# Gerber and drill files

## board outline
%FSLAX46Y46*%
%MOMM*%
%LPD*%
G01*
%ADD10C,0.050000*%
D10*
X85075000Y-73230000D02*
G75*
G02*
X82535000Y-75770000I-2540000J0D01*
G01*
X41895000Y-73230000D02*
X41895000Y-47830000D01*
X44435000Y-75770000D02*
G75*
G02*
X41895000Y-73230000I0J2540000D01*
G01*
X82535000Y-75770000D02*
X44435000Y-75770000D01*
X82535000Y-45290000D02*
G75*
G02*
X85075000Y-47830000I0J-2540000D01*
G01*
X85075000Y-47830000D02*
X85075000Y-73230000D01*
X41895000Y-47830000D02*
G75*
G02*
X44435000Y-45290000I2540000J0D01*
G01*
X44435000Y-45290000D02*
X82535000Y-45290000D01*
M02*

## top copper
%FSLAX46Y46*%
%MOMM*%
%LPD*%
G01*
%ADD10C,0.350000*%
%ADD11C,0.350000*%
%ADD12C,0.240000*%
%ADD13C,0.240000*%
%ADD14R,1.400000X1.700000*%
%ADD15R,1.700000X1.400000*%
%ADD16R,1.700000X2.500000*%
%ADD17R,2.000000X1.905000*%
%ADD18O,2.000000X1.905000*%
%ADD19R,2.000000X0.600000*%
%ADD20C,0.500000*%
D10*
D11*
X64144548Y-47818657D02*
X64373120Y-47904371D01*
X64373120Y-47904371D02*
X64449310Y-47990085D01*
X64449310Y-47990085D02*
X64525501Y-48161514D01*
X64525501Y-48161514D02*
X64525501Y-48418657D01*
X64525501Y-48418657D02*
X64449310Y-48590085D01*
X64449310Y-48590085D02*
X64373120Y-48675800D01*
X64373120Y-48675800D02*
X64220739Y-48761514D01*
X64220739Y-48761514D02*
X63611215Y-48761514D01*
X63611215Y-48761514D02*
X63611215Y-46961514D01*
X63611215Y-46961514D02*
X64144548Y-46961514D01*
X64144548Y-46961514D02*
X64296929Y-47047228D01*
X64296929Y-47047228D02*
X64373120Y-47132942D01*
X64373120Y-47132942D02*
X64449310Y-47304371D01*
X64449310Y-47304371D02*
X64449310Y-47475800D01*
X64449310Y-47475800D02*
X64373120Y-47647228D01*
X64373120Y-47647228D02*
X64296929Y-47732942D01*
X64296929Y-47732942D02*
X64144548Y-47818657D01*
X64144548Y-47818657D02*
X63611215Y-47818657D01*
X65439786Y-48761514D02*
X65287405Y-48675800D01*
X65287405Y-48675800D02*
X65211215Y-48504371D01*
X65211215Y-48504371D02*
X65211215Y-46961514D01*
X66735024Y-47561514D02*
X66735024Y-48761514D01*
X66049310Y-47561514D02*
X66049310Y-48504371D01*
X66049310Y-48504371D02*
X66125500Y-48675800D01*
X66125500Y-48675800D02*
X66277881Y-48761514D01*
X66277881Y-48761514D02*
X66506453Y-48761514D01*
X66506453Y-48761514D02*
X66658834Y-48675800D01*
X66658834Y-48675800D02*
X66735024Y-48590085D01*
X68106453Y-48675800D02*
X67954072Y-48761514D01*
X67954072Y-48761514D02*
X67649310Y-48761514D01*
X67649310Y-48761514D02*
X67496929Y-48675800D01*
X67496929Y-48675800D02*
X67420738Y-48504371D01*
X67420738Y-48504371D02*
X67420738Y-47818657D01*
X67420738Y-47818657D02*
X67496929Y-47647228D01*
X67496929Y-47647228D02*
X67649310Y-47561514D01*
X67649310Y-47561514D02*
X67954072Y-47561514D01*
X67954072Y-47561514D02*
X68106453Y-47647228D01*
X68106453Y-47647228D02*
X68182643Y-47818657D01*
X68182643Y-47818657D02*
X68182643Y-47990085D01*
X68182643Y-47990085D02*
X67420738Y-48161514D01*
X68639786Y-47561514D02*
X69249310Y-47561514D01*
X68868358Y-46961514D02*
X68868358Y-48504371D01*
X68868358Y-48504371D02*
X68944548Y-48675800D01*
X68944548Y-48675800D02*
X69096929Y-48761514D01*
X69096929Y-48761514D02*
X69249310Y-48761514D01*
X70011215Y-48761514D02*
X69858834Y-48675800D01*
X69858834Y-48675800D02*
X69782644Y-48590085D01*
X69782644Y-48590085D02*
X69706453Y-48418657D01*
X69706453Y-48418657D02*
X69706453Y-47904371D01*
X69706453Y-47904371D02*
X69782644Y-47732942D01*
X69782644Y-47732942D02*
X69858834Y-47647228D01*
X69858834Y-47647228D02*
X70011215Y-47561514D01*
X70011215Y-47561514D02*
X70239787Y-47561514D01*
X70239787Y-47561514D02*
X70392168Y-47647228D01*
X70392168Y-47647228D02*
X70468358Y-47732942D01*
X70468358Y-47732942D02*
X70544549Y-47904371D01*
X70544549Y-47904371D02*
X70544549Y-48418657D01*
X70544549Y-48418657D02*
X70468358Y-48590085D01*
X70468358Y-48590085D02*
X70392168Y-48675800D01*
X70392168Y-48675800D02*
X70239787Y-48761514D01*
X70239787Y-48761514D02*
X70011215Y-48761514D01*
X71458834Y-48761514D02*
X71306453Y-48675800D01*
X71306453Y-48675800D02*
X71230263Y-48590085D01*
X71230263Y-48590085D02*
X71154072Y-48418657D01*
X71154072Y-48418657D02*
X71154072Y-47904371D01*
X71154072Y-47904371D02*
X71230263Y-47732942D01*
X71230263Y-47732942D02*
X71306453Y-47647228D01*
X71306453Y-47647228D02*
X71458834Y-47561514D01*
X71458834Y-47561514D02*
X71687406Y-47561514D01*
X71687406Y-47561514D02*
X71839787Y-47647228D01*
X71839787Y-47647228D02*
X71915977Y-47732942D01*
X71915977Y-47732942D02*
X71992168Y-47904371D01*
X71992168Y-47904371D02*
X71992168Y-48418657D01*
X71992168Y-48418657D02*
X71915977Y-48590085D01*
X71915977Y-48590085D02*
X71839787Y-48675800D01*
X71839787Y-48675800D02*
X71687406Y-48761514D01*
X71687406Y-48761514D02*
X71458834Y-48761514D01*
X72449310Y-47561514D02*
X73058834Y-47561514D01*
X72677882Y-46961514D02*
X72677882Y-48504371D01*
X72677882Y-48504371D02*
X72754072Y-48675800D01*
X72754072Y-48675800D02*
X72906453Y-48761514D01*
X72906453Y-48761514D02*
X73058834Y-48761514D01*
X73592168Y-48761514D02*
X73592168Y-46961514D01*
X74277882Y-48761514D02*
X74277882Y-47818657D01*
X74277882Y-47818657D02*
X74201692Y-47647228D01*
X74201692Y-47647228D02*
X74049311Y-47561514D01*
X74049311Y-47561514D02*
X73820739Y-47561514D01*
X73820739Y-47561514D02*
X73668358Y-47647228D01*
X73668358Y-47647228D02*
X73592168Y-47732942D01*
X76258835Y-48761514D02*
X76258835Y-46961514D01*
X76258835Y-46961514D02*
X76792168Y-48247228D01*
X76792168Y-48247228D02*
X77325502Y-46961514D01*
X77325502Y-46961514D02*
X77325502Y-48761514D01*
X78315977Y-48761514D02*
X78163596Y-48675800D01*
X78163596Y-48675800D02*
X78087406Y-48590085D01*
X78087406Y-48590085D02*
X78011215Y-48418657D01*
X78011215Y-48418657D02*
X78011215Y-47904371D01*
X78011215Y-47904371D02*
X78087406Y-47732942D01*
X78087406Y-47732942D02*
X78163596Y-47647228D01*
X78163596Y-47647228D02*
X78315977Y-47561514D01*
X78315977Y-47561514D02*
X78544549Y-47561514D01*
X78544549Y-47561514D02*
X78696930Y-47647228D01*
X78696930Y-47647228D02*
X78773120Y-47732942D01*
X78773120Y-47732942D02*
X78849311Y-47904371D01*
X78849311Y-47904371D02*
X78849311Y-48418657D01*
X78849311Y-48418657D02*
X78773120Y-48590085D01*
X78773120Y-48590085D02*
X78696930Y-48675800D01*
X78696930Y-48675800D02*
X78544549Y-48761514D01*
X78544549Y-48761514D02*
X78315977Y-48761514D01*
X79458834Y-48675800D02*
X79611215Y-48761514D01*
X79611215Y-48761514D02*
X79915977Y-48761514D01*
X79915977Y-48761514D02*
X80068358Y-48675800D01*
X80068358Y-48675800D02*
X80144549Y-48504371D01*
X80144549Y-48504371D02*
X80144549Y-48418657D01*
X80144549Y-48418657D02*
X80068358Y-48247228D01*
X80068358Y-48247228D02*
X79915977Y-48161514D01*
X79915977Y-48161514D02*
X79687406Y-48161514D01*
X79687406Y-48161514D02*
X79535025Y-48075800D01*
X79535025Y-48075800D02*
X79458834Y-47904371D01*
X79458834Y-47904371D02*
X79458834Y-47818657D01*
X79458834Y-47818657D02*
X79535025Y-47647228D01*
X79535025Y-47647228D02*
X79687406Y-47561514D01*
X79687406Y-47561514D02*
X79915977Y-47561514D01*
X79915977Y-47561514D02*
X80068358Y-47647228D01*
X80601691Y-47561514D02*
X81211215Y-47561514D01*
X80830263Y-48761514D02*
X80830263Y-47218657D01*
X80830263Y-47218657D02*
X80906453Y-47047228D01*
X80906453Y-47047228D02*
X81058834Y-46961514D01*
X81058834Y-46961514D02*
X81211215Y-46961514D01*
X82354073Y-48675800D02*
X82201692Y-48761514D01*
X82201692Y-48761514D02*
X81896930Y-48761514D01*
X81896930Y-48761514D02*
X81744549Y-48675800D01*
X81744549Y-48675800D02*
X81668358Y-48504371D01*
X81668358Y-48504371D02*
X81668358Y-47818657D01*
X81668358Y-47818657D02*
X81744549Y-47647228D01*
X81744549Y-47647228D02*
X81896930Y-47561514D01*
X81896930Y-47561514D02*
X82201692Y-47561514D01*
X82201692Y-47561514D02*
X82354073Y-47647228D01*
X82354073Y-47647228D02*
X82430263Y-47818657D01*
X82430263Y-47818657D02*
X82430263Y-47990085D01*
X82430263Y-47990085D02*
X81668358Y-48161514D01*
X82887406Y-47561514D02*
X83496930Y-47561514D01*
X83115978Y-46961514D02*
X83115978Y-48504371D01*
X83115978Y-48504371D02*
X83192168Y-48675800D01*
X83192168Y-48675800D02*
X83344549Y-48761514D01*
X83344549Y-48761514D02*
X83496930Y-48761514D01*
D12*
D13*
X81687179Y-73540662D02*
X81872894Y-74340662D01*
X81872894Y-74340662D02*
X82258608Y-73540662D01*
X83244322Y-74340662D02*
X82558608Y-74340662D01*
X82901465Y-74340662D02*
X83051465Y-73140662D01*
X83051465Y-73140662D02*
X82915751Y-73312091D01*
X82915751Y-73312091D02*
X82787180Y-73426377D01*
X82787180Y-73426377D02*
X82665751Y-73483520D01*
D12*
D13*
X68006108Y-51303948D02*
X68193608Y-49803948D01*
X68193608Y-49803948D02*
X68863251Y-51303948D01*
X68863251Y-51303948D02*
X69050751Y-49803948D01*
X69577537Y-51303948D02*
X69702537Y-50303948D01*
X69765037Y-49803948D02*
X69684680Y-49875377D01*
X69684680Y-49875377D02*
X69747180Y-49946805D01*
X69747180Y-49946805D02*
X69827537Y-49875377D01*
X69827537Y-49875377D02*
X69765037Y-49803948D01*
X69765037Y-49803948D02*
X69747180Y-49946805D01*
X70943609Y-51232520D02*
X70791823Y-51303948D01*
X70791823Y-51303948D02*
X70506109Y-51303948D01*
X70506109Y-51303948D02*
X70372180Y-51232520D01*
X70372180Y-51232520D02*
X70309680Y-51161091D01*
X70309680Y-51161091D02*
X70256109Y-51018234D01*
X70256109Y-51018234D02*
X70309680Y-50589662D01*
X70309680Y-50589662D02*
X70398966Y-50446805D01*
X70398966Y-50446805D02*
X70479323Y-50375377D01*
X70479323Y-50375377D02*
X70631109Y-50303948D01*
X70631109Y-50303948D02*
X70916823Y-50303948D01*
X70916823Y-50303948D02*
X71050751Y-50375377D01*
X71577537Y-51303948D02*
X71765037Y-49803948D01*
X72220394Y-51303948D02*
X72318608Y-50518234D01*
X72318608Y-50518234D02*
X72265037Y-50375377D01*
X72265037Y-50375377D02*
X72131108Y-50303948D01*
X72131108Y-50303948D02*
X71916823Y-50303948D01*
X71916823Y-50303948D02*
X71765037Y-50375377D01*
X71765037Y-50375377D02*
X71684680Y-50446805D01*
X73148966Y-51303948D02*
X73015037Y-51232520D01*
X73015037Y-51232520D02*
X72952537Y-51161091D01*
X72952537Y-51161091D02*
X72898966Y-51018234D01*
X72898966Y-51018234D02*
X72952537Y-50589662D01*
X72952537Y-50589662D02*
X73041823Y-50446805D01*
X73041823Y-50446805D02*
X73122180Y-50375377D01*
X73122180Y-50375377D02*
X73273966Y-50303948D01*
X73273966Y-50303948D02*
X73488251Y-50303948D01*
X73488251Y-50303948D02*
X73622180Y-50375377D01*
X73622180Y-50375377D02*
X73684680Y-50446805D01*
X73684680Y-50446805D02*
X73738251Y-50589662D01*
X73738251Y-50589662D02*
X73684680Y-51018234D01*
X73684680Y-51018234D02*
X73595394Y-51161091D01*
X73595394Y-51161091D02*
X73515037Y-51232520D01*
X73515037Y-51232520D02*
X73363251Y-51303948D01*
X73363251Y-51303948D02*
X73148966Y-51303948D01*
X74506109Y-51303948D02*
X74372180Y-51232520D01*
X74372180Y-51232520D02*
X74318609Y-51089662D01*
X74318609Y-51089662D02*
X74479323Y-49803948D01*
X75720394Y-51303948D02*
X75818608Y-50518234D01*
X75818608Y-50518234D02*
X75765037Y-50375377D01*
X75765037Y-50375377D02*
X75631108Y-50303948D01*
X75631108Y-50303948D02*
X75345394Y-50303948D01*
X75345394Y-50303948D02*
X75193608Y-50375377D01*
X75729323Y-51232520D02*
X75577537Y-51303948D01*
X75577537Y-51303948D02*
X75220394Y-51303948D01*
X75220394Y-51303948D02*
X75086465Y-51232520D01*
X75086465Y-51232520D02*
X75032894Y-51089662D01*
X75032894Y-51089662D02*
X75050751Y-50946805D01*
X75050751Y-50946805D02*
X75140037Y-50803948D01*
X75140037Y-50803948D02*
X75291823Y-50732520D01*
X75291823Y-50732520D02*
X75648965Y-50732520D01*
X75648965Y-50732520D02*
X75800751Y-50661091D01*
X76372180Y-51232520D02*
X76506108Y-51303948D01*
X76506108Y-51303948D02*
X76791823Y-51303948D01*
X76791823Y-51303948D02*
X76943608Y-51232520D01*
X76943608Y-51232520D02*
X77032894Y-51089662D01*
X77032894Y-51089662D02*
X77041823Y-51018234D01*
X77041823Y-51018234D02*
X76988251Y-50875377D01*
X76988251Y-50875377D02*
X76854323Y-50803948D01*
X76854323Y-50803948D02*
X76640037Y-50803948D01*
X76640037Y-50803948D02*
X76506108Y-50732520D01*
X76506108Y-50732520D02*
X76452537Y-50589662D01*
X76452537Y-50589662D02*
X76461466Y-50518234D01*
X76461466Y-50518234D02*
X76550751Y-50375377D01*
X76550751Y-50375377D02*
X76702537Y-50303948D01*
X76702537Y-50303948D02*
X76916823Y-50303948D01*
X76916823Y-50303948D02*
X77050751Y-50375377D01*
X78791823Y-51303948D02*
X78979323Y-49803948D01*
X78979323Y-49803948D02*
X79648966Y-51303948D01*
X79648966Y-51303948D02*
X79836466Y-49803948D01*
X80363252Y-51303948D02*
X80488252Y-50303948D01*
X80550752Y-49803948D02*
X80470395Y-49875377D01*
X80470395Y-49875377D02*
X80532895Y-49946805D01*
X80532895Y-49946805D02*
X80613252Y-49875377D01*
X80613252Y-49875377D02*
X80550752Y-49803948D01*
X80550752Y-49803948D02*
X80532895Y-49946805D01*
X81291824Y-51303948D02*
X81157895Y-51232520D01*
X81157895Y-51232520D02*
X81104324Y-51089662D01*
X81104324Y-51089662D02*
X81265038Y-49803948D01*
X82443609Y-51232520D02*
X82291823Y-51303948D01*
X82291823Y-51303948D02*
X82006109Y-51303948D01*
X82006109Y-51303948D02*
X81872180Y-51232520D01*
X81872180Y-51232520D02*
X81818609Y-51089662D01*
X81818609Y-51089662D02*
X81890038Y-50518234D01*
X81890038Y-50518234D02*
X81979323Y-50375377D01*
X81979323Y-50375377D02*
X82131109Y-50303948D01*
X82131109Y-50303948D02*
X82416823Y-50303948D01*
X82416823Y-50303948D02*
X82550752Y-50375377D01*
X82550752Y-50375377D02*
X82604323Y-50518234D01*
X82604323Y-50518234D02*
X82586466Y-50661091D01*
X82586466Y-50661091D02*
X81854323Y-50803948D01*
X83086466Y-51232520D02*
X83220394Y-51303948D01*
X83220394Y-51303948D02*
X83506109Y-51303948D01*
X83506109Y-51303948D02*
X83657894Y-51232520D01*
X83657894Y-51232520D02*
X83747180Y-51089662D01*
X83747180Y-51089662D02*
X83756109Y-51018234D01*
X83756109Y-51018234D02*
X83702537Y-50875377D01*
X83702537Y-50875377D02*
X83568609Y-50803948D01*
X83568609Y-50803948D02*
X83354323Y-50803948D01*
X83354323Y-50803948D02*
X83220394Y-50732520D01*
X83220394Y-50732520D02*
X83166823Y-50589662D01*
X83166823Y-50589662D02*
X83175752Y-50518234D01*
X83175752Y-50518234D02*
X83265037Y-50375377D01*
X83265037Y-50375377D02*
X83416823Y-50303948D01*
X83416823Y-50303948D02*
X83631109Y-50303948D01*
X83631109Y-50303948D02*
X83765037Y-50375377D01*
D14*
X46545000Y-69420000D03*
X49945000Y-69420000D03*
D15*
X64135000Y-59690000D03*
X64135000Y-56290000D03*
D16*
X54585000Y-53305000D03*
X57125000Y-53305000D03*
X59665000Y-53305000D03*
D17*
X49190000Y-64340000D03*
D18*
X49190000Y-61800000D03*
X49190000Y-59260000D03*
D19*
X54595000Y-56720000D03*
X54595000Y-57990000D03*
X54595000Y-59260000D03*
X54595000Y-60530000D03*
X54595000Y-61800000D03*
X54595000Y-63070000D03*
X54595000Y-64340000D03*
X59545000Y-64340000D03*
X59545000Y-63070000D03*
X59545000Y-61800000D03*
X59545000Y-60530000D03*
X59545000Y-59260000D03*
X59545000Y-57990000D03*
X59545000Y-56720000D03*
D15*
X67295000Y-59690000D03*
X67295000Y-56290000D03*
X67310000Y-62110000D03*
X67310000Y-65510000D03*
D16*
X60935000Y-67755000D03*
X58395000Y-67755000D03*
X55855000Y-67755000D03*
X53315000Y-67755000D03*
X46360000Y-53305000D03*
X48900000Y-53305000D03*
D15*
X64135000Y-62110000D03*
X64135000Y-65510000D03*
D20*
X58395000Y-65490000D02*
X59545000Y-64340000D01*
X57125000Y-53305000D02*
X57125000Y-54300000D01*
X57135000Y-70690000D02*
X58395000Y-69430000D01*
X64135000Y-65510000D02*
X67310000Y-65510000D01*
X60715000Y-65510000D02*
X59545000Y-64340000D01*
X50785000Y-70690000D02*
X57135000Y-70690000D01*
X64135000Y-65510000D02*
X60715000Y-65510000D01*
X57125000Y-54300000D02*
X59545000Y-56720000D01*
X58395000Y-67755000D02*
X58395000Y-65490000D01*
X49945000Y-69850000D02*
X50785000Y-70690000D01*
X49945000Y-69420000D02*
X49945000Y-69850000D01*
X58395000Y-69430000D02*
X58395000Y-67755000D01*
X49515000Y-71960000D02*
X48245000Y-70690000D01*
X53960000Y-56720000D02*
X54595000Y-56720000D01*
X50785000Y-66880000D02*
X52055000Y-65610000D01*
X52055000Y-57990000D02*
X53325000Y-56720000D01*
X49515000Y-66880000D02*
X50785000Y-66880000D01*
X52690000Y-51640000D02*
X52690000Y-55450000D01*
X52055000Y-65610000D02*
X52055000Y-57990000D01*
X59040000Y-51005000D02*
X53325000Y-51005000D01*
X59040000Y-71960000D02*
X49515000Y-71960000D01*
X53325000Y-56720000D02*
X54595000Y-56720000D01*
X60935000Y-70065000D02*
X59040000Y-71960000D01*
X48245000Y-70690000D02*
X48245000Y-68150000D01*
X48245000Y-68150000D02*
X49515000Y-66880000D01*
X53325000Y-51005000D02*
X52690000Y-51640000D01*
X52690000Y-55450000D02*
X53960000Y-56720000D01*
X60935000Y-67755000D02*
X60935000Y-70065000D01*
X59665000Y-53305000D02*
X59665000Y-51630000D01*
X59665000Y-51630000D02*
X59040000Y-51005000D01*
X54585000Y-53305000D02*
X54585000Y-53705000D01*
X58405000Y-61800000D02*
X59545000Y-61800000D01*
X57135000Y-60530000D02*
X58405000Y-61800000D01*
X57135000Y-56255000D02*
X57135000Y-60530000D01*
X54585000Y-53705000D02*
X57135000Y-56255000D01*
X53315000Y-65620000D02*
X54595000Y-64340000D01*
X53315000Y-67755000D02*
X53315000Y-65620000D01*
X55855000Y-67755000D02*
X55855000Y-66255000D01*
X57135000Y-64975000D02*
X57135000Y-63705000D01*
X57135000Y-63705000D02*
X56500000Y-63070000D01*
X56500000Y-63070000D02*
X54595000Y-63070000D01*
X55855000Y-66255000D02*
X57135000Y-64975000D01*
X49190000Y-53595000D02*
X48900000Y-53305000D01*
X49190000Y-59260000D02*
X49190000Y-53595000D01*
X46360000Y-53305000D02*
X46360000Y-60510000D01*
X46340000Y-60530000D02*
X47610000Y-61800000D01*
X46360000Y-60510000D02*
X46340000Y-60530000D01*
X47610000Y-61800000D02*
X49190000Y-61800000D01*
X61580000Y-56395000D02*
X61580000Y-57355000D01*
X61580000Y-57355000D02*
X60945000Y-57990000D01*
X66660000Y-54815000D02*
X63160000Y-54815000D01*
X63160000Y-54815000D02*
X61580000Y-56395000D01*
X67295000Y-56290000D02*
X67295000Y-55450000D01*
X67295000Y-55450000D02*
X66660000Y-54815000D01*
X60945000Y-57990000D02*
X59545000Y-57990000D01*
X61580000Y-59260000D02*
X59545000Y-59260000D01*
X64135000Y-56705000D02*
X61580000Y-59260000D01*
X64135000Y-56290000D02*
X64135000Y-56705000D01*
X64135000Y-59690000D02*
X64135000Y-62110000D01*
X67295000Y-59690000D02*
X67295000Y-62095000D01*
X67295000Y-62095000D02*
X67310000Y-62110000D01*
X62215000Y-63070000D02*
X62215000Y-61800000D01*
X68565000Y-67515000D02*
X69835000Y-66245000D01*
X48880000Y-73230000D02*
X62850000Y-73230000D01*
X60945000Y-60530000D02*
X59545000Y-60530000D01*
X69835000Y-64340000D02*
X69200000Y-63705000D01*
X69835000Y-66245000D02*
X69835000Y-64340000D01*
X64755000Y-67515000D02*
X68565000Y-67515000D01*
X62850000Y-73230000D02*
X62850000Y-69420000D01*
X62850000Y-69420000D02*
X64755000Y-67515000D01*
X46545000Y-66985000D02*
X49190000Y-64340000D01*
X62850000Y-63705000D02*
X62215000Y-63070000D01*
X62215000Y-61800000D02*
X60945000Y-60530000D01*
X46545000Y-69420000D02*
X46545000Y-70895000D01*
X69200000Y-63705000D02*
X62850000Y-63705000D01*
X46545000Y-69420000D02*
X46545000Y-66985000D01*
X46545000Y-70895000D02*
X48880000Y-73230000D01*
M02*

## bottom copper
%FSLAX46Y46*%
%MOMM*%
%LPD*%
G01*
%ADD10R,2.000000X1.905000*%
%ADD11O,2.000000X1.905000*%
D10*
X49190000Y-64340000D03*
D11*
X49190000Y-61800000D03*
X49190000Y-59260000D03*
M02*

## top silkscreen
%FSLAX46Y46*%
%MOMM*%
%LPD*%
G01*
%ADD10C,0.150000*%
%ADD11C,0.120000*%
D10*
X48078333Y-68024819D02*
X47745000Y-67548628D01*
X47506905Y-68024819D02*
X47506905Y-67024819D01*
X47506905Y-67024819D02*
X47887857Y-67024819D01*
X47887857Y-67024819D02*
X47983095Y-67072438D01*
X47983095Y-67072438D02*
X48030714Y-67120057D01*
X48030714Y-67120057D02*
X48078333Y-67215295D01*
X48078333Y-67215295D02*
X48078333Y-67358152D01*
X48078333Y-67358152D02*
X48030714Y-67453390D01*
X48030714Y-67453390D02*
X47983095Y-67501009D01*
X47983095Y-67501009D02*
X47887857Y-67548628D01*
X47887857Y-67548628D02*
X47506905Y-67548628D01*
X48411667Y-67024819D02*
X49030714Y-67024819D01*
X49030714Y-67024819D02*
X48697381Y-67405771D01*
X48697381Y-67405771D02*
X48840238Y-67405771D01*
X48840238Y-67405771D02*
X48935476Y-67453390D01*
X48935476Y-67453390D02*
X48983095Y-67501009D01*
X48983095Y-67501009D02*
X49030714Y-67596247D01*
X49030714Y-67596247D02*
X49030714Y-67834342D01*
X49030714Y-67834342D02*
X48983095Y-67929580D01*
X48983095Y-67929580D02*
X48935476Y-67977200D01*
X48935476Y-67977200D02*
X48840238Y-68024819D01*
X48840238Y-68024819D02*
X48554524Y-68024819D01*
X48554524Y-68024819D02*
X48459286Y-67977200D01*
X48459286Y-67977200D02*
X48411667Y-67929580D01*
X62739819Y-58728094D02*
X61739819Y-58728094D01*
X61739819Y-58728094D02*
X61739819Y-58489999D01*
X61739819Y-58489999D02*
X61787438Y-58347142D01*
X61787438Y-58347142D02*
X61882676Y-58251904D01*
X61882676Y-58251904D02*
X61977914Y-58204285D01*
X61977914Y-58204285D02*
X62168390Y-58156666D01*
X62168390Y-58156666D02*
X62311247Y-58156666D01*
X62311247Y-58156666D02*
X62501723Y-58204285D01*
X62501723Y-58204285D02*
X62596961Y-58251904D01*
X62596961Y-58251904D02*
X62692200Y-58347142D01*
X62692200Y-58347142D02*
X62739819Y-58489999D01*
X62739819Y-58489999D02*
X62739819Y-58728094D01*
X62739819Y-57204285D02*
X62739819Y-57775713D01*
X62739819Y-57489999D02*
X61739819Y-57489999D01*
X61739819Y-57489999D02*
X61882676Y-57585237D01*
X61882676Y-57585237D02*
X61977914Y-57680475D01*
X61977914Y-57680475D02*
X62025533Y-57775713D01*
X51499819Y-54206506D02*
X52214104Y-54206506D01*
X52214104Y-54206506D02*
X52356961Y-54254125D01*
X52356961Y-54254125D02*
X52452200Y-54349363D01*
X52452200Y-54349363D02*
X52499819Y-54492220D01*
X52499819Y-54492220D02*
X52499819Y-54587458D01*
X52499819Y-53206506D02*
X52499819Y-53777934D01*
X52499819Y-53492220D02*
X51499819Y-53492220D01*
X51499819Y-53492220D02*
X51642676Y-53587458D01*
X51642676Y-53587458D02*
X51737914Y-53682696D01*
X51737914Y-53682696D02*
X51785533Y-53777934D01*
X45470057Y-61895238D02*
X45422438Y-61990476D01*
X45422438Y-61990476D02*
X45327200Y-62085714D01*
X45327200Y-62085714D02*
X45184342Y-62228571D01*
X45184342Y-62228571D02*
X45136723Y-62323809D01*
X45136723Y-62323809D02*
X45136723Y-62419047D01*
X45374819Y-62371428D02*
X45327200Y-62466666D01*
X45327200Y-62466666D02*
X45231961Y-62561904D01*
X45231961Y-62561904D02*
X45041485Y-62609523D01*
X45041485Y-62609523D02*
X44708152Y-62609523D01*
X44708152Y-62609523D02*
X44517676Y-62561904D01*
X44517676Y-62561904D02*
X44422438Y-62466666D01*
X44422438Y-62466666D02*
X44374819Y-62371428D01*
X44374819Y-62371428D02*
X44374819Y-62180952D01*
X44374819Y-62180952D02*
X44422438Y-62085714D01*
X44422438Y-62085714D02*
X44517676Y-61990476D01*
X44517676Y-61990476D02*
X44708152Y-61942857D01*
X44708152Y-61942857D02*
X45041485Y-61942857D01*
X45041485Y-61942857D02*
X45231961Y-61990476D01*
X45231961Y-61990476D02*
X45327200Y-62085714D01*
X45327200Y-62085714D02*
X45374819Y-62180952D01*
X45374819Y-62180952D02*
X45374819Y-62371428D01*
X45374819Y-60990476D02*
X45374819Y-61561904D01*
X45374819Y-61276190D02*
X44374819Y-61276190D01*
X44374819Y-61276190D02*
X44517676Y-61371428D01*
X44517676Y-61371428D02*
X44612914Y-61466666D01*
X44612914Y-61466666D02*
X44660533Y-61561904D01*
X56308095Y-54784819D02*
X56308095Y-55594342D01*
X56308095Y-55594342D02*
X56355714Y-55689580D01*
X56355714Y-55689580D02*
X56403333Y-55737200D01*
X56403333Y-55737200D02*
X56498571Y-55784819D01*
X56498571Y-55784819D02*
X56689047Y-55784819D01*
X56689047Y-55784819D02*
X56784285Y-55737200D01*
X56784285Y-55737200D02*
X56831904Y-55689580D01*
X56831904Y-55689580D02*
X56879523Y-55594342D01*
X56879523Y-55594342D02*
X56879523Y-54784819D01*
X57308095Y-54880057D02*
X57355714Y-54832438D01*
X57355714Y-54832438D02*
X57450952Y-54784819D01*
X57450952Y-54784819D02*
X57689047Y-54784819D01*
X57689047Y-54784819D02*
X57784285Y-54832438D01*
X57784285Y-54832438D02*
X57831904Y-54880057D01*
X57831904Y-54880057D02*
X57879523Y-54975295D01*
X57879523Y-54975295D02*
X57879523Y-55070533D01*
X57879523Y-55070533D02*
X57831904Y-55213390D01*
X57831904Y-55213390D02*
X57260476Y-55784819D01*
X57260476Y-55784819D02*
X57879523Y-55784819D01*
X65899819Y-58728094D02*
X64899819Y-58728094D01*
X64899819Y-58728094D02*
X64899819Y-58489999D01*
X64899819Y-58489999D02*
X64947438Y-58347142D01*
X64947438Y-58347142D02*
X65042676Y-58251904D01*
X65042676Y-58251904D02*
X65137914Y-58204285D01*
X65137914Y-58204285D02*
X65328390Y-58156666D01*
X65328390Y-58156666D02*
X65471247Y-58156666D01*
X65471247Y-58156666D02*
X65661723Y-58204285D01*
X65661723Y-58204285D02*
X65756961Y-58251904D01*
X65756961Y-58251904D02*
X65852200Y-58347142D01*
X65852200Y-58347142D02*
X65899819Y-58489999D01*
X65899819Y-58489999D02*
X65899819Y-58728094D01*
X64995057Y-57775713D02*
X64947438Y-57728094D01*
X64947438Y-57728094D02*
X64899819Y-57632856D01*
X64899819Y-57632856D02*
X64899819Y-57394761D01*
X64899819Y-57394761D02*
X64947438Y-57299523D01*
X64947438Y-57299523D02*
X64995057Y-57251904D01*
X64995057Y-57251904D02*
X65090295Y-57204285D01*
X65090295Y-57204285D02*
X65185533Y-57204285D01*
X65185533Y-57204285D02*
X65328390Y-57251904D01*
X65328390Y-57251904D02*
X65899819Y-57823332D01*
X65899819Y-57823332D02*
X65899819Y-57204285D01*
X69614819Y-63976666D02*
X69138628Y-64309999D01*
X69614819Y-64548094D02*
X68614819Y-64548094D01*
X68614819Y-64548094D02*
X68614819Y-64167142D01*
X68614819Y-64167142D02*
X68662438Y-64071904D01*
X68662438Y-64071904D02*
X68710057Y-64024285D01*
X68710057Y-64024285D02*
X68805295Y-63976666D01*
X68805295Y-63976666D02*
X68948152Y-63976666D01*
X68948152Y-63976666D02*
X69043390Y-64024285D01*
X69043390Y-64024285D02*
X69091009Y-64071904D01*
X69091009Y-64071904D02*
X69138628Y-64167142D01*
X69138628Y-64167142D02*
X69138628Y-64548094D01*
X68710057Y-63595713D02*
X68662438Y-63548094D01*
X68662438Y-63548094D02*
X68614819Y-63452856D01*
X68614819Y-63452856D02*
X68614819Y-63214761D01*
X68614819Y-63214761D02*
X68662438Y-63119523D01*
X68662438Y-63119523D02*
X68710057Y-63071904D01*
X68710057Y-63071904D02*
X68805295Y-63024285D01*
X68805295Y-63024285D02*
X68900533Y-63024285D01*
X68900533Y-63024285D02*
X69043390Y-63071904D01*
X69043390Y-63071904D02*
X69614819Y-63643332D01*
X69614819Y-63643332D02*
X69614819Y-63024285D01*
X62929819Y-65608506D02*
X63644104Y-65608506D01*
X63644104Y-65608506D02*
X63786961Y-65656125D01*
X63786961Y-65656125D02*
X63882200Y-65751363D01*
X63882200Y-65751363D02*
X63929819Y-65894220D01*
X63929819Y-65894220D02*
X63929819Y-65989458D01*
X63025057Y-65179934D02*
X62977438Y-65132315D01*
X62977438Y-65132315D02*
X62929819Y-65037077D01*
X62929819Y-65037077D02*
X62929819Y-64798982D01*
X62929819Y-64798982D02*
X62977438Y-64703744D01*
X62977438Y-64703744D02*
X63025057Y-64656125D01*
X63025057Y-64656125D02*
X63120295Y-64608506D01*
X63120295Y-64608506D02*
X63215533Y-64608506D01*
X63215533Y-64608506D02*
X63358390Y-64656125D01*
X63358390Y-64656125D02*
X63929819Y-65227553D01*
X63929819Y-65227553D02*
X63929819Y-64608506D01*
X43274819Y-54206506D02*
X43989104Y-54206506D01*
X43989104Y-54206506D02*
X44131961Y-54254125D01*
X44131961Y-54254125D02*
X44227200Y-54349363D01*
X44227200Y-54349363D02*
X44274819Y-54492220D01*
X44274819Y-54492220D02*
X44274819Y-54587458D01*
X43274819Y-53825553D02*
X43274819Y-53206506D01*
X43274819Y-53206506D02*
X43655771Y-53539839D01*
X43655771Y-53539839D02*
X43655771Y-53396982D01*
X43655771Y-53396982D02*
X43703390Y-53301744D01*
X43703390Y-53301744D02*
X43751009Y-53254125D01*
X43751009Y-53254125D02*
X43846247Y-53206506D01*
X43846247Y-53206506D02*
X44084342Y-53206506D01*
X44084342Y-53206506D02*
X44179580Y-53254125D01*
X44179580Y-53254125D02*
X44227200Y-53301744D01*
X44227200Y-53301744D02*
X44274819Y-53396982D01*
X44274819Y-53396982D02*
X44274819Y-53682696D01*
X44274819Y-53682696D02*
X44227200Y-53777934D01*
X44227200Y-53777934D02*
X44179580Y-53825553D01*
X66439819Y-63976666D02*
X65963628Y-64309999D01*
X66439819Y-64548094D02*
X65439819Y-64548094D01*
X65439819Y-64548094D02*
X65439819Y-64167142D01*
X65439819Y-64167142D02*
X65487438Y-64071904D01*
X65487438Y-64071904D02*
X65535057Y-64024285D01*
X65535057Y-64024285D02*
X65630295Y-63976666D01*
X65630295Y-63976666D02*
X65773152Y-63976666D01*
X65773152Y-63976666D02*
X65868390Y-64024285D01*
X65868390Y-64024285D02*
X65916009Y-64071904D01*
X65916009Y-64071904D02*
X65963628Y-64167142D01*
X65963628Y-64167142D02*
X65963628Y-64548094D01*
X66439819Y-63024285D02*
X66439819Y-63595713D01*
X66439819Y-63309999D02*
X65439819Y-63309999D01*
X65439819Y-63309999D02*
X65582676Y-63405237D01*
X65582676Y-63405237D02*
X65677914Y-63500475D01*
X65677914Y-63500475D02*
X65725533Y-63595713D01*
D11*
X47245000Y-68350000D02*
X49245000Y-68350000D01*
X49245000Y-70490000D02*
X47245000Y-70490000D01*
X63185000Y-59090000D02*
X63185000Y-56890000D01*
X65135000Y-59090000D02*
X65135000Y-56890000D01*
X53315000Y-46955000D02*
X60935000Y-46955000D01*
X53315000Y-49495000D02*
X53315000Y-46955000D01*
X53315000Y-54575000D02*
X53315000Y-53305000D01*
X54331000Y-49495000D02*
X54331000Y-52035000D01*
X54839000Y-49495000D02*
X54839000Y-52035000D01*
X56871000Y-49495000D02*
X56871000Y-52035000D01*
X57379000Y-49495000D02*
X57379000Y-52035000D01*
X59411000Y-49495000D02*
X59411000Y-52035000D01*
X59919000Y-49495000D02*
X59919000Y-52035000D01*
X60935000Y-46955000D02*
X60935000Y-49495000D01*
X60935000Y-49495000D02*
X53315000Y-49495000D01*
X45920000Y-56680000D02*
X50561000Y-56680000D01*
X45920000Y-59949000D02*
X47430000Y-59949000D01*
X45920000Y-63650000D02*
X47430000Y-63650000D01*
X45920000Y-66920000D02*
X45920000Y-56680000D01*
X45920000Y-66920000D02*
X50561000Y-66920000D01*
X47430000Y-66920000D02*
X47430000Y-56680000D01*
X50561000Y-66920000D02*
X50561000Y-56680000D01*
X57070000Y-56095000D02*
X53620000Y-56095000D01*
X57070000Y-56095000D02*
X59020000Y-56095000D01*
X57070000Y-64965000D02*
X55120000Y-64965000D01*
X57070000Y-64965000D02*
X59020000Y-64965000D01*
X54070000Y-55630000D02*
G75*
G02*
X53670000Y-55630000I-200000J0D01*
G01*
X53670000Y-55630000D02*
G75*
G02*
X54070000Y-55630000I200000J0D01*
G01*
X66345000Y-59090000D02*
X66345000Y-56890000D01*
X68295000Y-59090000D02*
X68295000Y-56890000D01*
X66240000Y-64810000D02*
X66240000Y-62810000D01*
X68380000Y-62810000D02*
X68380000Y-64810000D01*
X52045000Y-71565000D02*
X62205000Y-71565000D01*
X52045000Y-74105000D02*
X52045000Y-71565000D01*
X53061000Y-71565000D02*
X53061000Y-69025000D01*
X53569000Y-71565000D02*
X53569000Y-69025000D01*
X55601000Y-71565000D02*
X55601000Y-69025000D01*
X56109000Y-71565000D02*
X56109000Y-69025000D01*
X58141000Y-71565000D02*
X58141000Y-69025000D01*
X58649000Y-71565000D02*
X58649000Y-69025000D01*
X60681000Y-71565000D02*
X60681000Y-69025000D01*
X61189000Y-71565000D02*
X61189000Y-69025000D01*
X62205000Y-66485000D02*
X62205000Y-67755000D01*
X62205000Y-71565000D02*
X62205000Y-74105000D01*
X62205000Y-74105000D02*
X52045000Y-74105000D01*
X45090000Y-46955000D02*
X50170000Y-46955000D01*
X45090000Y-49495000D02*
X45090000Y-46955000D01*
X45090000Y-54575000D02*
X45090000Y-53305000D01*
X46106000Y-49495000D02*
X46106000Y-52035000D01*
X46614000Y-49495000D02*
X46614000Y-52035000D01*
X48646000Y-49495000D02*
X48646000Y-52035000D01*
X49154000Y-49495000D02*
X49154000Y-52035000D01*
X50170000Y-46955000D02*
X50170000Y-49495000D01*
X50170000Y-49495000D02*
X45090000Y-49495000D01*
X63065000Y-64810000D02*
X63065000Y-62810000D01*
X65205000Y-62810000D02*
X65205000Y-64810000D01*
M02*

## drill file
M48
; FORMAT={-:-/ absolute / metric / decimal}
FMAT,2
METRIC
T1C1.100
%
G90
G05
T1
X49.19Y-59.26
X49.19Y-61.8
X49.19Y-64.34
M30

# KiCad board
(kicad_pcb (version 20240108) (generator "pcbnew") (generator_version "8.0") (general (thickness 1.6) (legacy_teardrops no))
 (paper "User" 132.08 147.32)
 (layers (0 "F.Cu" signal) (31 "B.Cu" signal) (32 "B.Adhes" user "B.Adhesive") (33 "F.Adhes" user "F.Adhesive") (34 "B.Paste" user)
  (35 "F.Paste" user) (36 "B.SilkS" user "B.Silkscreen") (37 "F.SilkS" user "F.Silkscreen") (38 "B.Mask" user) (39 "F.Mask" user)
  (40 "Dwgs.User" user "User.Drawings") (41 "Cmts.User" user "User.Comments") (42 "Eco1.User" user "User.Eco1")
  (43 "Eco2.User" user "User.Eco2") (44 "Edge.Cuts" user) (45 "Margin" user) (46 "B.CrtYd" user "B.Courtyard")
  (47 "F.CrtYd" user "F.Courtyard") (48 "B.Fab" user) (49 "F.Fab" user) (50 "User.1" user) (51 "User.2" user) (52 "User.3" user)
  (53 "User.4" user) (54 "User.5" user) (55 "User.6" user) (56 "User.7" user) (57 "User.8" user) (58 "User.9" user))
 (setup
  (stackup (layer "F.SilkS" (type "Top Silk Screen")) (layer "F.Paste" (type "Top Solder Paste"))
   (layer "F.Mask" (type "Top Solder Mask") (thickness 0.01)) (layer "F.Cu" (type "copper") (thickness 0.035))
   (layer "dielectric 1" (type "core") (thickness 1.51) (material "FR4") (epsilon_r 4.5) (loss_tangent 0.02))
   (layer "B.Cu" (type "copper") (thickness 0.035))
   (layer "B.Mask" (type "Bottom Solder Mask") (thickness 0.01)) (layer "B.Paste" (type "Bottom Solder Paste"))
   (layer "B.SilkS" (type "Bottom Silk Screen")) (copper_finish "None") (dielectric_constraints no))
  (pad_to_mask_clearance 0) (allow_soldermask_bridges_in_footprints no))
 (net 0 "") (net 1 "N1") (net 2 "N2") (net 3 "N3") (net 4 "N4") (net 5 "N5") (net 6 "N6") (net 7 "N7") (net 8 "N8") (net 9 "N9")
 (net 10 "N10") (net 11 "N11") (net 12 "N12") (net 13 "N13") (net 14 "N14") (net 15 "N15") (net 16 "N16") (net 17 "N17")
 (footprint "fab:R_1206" (layer "F.Cu") (at 48.245 69.42)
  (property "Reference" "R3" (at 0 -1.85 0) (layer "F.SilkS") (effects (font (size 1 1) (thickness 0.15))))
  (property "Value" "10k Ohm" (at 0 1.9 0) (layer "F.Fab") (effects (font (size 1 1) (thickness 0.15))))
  (fp_line (start -1 -1.07) (end 1 -1.07) (stroke (width 0.12) (type solid)) (layer "F.SilkS"))
  (fp_line (start 1 1.07) (end -1 1.07) (stroke (width 0.12) (type solid)) (layer "F.SilkS"))
  (pad "1" smd rect (at -1.7 0) (size 1.4 1.7) (layers "F.Cu" "F.Paste" "F.Mask") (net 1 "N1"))
  (pad "2" smd rect (at 1.7 0) (size 1.4 1.7) (layers "F.Cu" "F.Paste" "F.Mask") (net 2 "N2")))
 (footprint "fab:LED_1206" (layer "F.Cu") (at 64.135 57.99 90)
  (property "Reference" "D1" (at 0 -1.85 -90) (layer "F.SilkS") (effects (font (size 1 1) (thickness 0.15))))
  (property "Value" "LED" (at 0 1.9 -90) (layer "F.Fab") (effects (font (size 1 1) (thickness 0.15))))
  (fp_line (start -1.1 -0.95) (end 1.1 -0.95) (stroke (width 0.12) (type solid)) (layer "F.SilkS"))
  (fp_line (start -1.1 1) (end 1.1 1) (stroke (width 0.12) (type solid)) (layer "F.SilkS"))
  (pad "1" smd rect (at -1.7 0 90) (size 1.4 1.7) (layers "F.Cu" "F.Paste" "F.Mask") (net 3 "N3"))
  (pad "2" smd rect (at 1.7 0 90) (size 1.4 1.7) (layers "F.Cu" "F.Paste" "F.Mask") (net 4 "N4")))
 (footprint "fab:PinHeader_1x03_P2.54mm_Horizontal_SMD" (layer "F.Cu") (at 54.585 53.305 90)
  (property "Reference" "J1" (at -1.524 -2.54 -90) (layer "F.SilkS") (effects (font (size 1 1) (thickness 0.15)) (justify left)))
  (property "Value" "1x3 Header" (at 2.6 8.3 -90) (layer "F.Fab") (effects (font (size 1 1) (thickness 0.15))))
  (fp_line (start 6.35 -1.27) (end 6.35 6.35) (stroke (width 0.12) (type solid)) (layer "F.SilkS"))
  (fp_line (start 3.81 -1.27) (end 6.35 -1.27) (stroke (width 0.12) (type solid)) (layer "F.SilkS"))
  (fp_line (start -1.27 -1.27) (end 0 -1.27) (stroke (width 0.12) (type solid)) (layer "F.SilkS"))
  (fp_line (start 3.81 -0.254) (end 1.27 -0.254) (stroke (width 0.12) (type solid)) (layer "F.SilkS"))
  (fp_line (start 3.81 0.254) (end 1.27 0.254) (stroke (width 0.12) (type solid)) (layer "F.SilkS"))
  (fp_line (start 3.81 2.286) (end 1.27 2.286) (stroke (width 0.12) (type solid)) (layer "F.SilkS"))
  (fp_line (start 3.81 2.794) (end 1.27 2.794) (stroke (width 0.12) (type solid)) (layer "F.SilkS"))
  (fp_line (start 3.81 4.826) (end 1.27 4.826) (stroke (width 0.12) (type solid)) (layer "F.SilkS"))
  (fp_line (start 3.81 5.334) (end 1.27 5.334) (stroke (width 0.12) (type solid)) (layer "F.SilkS"))
  (fp_line (start 6.35 6.35) (end 3.81 6.35) (stroke (width 0.12) (type solid)) (layer "F.SilkS"))
  (fp_line (start 3.81 6.35) (end 3.81 -1.27) (stroke (width 0.12) (type solid)) (layer "F.SilkS"))
  (pad "1" smd rect (at 0 0 90) (size 2.5 1.7) (layers "F.Cu" "F.Paste" "F.Mask") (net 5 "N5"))
  (pad "2" smd rect (at 0 2.54 90) (size 2.5 1.7) (layers "F.Cu" "F.Paste" "F.Mask") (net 2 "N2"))
  (pad "3" smd rect (at 0 5.08 90) (size 2.5 1.7) (layers "F.Cu" "F.Paste" "F.Mask") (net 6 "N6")))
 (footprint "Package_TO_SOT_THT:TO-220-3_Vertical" (layer "F.Cu") (at 49.19 64.34 90)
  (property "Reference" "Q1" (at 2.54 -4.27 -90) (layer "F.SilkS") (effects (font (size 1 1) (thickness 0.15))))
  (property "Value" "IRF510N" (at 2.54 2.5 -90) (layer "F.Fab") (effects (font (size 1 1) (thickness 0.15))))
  (fp_line (start 7.66 -3.27) (end 7.66 1.371) (stroke (width 0.12) (type solid)) (layer "F.SilkS"))
  (fp_line (start 4.391 -3.27) (end 4.391 -1.76) (stroke (width 0.12) (type solid)) (layer "F.SilkS"))
  (fp_line (start 0.69 -3.27) (end 0.69 -1.76) (stroke (width 0.12) (type solid)) (layer "F.SilkS"))
  (fp_line (start -2.58 -3.27) (end 7.66 -3.27) (stroke (width 0.12) (type solid)) (layer "F.SilkS"))
  (fp_line (start -2.58 -3.27) (end -2.58 1.371) (stroke (width 0.12) (type solid)) (layer "F.SilkS"))
  (fp_line (start -2.58 -1.76) (end 7.66 -1.76) (stroke (width 0.12) (type solid)) (layer "F.SilkS"))
  (fp_line (start -2.58 1.371) (end 7.66 1.371) (stroke (width 0.12) (type solid)) (layer "F.SilkS"))
  (pad "1" thru_hole rect (at 0 0 90) (size 1.905 2) (drill 1.1) (layers "*.Cu" "*.Mask") (remove_unused_layers no) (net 1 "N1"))
  (pad "2" thru_hole oval (at 2.54 0 90) (size 1.905 2) (drill 1.1) (layers "*.Cu" "*.Mask") (remove_unused_layers no) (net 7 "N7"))
  (pad "3" thru_hole oval (at 5.08 0 90) (size 1.905 2) (drill 1.1) (layers "*.Cu" "*.Mask") (remove_unused_layers no) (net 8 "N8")))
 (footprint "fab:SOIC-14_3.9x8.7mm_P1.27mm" (layer "F.Cu") (at 57.07 60.53)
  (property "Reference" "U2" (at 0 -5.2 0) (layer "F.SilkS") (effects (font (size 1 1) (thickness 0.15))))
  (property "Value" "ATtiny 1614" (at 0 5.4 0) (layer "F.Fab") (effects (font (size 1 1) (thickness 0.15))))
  (fp_line (start 0 -4.435) (end -3.45 -4.435) (stroke (width 0.12) (type solid)) (layer "F.SilkS"))
  (fp_line (start 0 -4.435) (end 1.95 -4.435) (stroke (width 0.12) (type solid)) (layer "F.SilkS"))
  (fp_line (start 0 4.435) (end -1.95 4.435) (stroke (width 0.12) (type solid)) (layer "F.SilkS"))
  (fp_line (start 0 4.435) (end 1.95 4.435) (stroke (width 0.12) (type solid)) (layer "F.SilkS"))
  (fp_circle (center -3.2 -4.9) (end -3.2 -4.7) (stroke (width 0.12) (type solid)) (fill none) (layer "F.SilkS"))
  (pad "1" smd rect (at -2.475 -3.81) (size 2 0.6) (layers "F.Cu" "F.Paste" "F.Mask") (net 6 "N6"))
  (pad "2" smd rect (at -2.475 -2.54) (size 2 0.6) (layers "F.Cu" "F.Paste" "F.Mask") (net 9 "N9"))
  (pad "3" smd rect (at -2.475 -1.27) (size 2 0.6) (layers "F.Cu" "F.Paste" "F.Mask") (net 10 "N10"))
  (pad "4" smd rect (at -2.475 0) (size 2 0.6) (layers "F.Cu" "F.Paste" "F.Mask") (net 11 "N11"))
  (pad "5" smd rect (at -2.475 1.27) (size 2 0.6) (layers "F.Cu" "F.Paste" "F.Mask") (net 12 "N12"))
  (pad "6" smd rect (at -2.475 2.54) (size 2 0.6) (layers "F.Cu" "F.Paste" "F.Mask") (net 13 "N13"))
  (pad "7" smd rect (at -2.475 3.81) (size 2 0.6) (layers "F.Cu" "F.Paste" "F.Mask") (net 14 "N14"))
  (pad "8" smd rect (at 2.475 3.81) (size 2 0.6) (layers "F.Cu" "F.Paste" "F.Mask") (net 2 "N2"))
  (pad "9" smd rect (at 2.475 2.54) (size 2 0.6) (layers "F.Cu" "F.Paste" "F.Mask") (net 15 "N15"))
  (pad "10" smd rect (at 2.475 1.27) (size 2 0.6) (layers "F.Cu" "F.Paste" "F.Mask") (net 5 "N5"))
  (pad "11" smd rect (at 2.475 0) (size 2 0.6) (layers "F.Cu" "F.Paste" "F.Mask") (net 1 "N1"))
  (pad "12" smd rect (at 2.475 -1.27) (size 2 0.6) (layers "F.Cu" "F.Paste" "F.Mask") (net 4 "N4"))
  (pad "13" smd rect (at 2.475 -2.54) (size 2 0.6) (layers "F.Cu" "F.Paste" "F.Mask") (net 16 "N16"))
  (pad "14" smd rect (at 2.475 -3.81) (size 2 0.6) (layers "F.Cu" "F.Paste" "F.Mask") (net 2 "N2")))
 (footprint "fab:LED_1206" (layer "F.Cu") (at 67.295 57.99 90)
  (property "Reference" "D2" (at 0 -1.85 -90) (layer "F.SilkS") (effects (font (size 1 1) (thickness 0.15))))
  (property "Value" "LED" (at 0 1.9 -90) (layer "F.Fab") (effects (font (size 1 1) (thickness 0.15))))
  (fp_line (start -1.1 -0.95) (end 1.1 -0.95) (stroke (width 0.12) (type solid)) (layer "F.SilkS"))
  (fp_line (start -1.1 1) (end 1.1 1) (stroke (width 0.12) (type solid)) (layer "F.SilkS"))
  (pad "1" smd rect (at -1.7 0 90) (size 1.4 1.7) (layers "F.Cu" "F.Paste" "F.Mask") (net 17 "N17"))
  (pad "2" smd rect (at 1.7 0 90) (size 1.4 1.7) (layers "F.Cu" "F.Paste" "F.Mask") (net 16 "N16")))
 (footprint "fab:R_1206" (layer "F.Cu") (at 67.31 63.81 -90)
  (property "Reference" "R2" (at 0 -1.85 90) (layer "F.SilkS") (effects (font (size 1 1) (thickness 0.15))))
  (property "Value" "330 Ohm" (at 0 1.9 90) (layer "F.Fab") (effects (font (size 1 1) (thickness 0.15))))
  (fp_line (start 1 1.07) (end -1 1.07) (stroke (width 0.12) (type solid)) (layer "F.SilkS"))
  (fp_line (start -1 -1.07) (end 1 -1.07) (stroke (width 0.12) (type solid)) (layer "F.SilkS"))
  (pad "1" smd rect (at -1.7 0 270) (size 1.4 1.7) (layers "F.Cu" "F.Paste" "F.Mask") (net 17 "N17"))
  (pad "2" smd rect (at 1.7 0 270) (size 1.4 1.7) (layers "F.Cu" "F.Paste" "F.Mask") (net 2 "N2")))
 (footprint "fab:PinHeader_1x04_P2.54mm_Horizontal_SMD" (layer "F.Cu") (at 60.935 67.755 -90)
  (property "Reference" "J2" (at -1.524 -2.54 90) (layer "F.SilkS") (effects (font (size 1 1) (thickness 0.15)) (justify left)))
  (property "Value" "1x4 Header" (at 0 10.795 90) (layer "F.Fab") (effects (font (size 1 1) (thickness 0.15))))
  (fp_line (start 3.81 8.89) (end 3.81 -1.27) (stroke (width 0.12) (type solid)) (layer "F.SilkS"))
  (fp_line (start 6.35 8.89) (end 3.81 8.89) (stroke (width 0.12) (type solid)) (layer "F.SilkS"))
  (fp_line (start 3.81 7.874) (end 1.27 7.874) (stroke (width 0.12) (type solid)) (layer "F.SilkS"))
  (fp_line (start 3.81 7.366) (end 1.27 7.366) (stroke (width 0.12) (type solid)) (layer "F.SilkS"))
  (fp_line (start 3.81 5.334) (end 1.27 5.334) (stroke (width 0.12) (type solid)) (layer "F.SilkS"))
  (fp_line (start 3.81 4.826) (end 1.27 4.826) (stroke (width 0.12) (type solid)) (layer "F.SilkS"))
  (fp_line (start 3.81 2.794) (end 1.27 2.794) (stroke (width 0.12) (type solid)) (layer "F.SilkS"))
  (fp_line (start 3.81 2.286) (end 1.27 2.286) (stroke (width 0.12) (type solid)) (layer "F.SilkS"))
  (fp_line (start 3.81 0.254) (end 1.27 0.254) (stroke (width 0.12) (type solid)) (layer "F.SilkS"))
  (fp_line (start 3.81 -0.254) (end 1.27 -0.254) (stroke (width 0.12) (type solid)) (layer "F.SilkS"))
  (fp_line (start -1.27 -1.27) (end 0 -1.27) (stroke (width 0.12) (type solid)) (layer "F.SilkS"))
  (fp_line (start 3.81 -1.27) (end 6.35 -1.27) (stroke (width 0.12) (type solid)) (layer "F.SilkS"))
  (fp_line (start 6.35 -1.27) (end 6.35 8.89) (stroke (width 0.12) (type solid)) (layer "F.SilkS"))
  (pad "1" smd rect (at 0 0 270) (size 2.5 1.7) (layers "F.Cu" "F.Paste" "F.Mask") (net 6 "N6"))
  (pad "2" smd rect (at 0 2.54 270) (size 2.5 1.7) (layers "F.Cu" "F.Paste" "F.Mask") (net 2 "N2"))
  (pad "3" smd rect (at 0 5.08 270) (size 2.5 1.7) (layers "F.Cu" "F.Paste" "F.Mask") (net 13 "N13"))
  (pad "4" smd rect (at 0 7.62 270) (size 2.5 1.7) (layers "F.Cu" "F.Paste" "F.Mask") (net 14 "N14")))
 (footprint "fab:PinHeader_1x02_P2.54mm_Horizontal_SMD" (layer "F.Cu") (at 46.36 53.305 90)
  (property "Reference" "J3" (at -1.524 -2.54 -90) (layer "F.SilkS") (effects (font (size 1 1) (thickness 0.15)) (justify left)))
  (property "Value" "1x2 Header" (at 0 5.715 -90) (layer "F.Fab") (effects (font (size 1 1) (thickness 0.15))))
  (fp_line (start 6.35 -1.27) (end 6.35 3.81) (stroke (width 0.12) (type solid)) (layer "F.SilkS"))
  (fp_line (start 3.81 -1.27) (end 6.35 -1.27) (stroke (width 0.12) (type solid)) (layer "F.SilkS"))
  (fp_line (start -1.27 -1.27) (end 0 -1.27) (stroke (width 0.12) (type solid)) (layer "F.SilkS"))
  (fp_line (start 3.81 -0.254) (end 1.27 -0.254) (stroke (width 0.12) (type solid)) (layer "F.SilkS"))
  (fp_line (start 3.81 0.254) (end 1.27 0.254) (stroke (width 0.12) (type solid)) (layer "F.SilkS"))
  (fp_line (start 3.81 2.286) (end 1.27 2.286) (stroke (width 0.12) (type solid)) (layer "F.SilkS"))
  (fp_line (start 3.81 2.794) (end 1.27 2.794) (stroke (width 0.12) (type solid)) (layer "F.SilkS"))
  (fp_line (start 6.35 3.81) (end 3.81 3.81) (stroke (width 0.12) (type solid)) (layer "F.SilkS"))
  (fp_line (start 3.81 3.81) (end 3.81 -1.27) (stroke (width 0.12) (type solid)) (layer "F.SilkS"))
  (pad "1" smd rect (at 0 0 90) (size 2.5 1.7) (layers "F.Cu" "F.Paste" "F.Mask") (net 7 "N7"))
  (pad "2" smd rect (at 0 2.54 90) (size 2.5 1.7) (layers "F.Cu" "F.Paste" "F.Mask") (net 8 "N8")))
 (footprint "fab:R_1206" (layer "F.Cu") (at 64.135 63.81 -90)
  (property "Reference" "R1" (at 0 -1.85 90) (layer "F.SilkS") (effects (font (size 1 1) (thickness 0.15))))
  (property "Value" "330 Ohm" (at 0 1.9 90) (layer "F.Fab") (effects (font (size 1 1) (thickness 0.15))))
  (fp_line (start 1 1.07) (end -1 1.07) (stroke (width 0.12) (type solid)) (layer "F.SilkS"))
  (fp_line (start -1 -1.07) (end 1 -1.07) (stroke (width 0.12) (type solid)) (layer "F.SilkS"))
  (pad "1" smd rect (at -1.7 0 270) (size 1.4 1.7) (layers "F.Cu" "F.Paste" "F.Mask") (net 3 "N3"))
  (pad "2" smd rect (at 1.7 0 270) (size 1.4 1.7) (layers "F.Cu" "F.Paste" "F.Mask") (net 2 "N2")))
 (gr_arc (start 85.075 73.23) (mid 84.331051 75.026051) (end 82.535 75.77) (stroke (width 0.05) (type default)) (layer "Edge.Cuts"))
 (gr_line (start 41.895 73.23) (end 41.895 47.83) (stroke (width 0.05) (type default)) (layer "Edge.Cuts"))
 (gr_arc (start 44.435 75.77) (mid 42.638949 75.026051) (end 41.895 73.23) (stroke (width 0.05) (type default)) (layer "Edge.Cuts"))
 (gr_line (start 82.535 75.77) (end 44.435 75.77) (stroke (width 0.05) (type default)) (layer "Edge.Cuts"))
 (gr_arc (start 82.535 45.29) (mid 84.331051 46.033949) (end 85.075 47.83) (stroke (width 0.05) (type default)) (layer "Edge.Cuts"))
 (gr_line (start 85.075 47.83) (end 85.075 73.23) (stroke (width 0.05) (type default)) (layer "Edge.Cuts"))
 (gr_arc (start 41.895 47.83) (mid 42.638949 46.033949) (end 44.435 45.29) (stroke (width 0.05) (type default)) (layer "Edge.Cuts"))
 (gr_line (start 44.435 45.29) (end 82.535 45.29) (stroke (width 0.05) (type default)) (layer "Edge.Cuts"))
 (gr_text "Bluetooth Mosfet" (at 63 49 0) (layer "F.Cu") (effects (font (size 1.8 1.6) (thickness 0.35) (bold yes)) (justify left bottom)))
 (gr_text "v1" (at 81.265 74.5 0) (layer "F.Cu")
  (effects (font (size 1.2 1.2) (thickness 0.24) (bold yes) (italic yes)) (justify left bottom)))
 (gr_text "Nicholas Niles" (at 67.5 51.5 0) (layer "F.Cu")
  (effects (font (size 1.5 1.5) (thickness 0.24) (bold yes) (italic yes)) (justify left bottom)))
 (segment (start 58.395 65.49) (end 59.545 64.34) (width 0.5) (layer "F.Cu") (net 2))
 (segment (start 57.125 53.305) (end 57.125 54.3) (width 0.5) (layer "F.Cu") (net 2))
 (segment (start 57.135 70.69) (end 58.395 69.43) (width 0.5) (layer "F.Cu") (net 2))
 (segment (start 64.135 65.51) (end 67.31 65.51) (width 0.5) (layer "F.Cu") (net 2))
 (segment (start 60.715 65.51) (end 59.545 64.34) (width 0.5) (layer "F.Cu") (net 2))
 (segment (start 50.785 70.69) (end 57.135 70.69) (width 0.5) (layer "F.Cu") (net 2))
 (segment (start 64.135 65.51) (end 60.715 65.51) (width 0.5) (layer "F.Cu") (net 2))
 (segment (start 57.125 54.3) (end 59.545 56.72) (width 0.5) (layer "F.Cu") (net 2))
 (segment (start 58.395 67.755) (end 58.395 65.49) (width 0.5) (layer "F.Cu") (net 2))
 (segment (start 49.945 69.85) (end 50.785 70.69) (width 0.5) (layer "F.Cu") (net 2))
 (segment (start 49.945 69.42) (end 49.945 69.85) (width 0.5) (layer "F.Cu") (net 2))
 (segment (start 58.395 69.43) (end 58.395 67.755) (width 0.5) (layer "F.Cu") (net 2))
 (segment (start 49.515 71.96) (end 48.245 70.69) (width 0.5) (layer "F.Cu") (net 6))
 (segment (start 53.96 56.72) (end 54.595 56.72) (width 0.5) (layer "F.Cu") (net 6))
 (segment (start 50.785 66.88) (end 52.055 65.61) (width 0.5) (layer "F.Cu") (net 6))
 (segment (start 52.055 57.99) (end 53.325 56.72) (width 0.5) (layer "F.Cu") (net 6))
 (segment (start 49.515 66.88) (end 50.785 66.88) (width 0.5) (layer "F.Cu") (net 6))
 (segment (start 52.69 51.64) (end 52.69 55.45) (width 0.5) (layer "F.Cu") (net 6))
 (segment (start 52.055 65.61) (end 52.055 57.99) (width 0.5) (layer "F.Cu") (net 6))
 (segment (start 59.04 51.005) (end 53.325 51.005) (width 0.5) (layer "F.Cu") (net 6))
 (segment (start 59.04 71.96) (end 49.515 71.96) (width 0.5) (layer "F.Cu") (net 6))
 (segment (start 53.325 56.72) (end 54.595 56.72) (width 0.5) (layer "F.Cu") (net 6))
 (segment (start 60.935 70.065) (end 59.04 71.96) (width 0.5) (layer "F.Cu") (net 6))
 (segment (start 48.245 70.69) (end 48.245 68.15) (width 0.5) (layer "F.Cu") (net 6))
 (segment (start 48.245 68.15) (end 49.515 66.88) (width 0.5) (layer "F.Cu") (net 6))
 (segment (start 53.325 51.005) (end 52.69 51.64) (width 0.5) (layer "F.Cu") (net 6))
 (segment (start 52.69 55.45) (end 53.96 56.72) (width 0.5) (layer "F.Cu") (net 6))
 (segment (start 60.935 67.755) (end 60.935 70.065) (width 0.5) (layer "F.Cu") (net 6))
 (segment (start 59.665 53.305) (end 59.665 51.63) (width 0.5) (layer "F.Cu") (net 6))
 (segment (start 59.665 51.63) (end 59.04 51.005) (width 0.5) (layer "F.Cu") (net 6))
 (segment (start 54.585 53.305) (end 54.585 53.705) (width 0.5) (layer "F.Cu") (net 5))
 (segment (start 58.405 61.8) (end 59.545 61.8) (width 0.5) (layer "F.Cu") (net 5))
 (segment (start 57.135 60.53) (end 58.405 61.8) (width 0.5) (layer "F.Cu") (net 5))
 (segment (start 57.135 56.255) (end 57.135 60.53) (width 0.5) (layer "F.Cu") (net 5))
 (segment (start 54.585 53.705) (end 57.135 56.255) (width 0.5) (layer "F.Cu") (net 5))
 (segment (start 53.315 65.62) (end 54.595 64.34) (width 0.5) (layer "F.Cu") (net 14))
 (segment (start 53.315 67.755) (end 53.315 65.62) (width 0.5) (layer "F.Cu") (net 14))
 (segment (start 55.855 67.755) (end 55.855 66.255) (width 0.5) (layer "F.Cu") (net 13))
 (segment (start 57.135 64.975) (end 57.135 63.705) (width 0.5) (layer "F.Cu") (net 13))
 (segment (start 57.135 63.705) (end 56.5 63.07) (width 0.5) (layer "F.Cu") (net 13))
 (segment (start 56.5 63.07) (end 54.595 63.07) (width 0.5) (layer "F.Cu") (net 13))
 (segment (start 55.855 66.255) (end 57.135 64.975) (width 0.5) (layer "F.Cu") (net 13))
 (segment (start 49.19 53.595) (end 48.9 53.305) (width 0.5) (layer "F.Cu") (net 8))
 (segment (start 49.19 59.26) (end 49.19 53.595) (width 0.5) (layer "F.Cu") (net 8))
 (segment (start 46.36 53.305) (end 46.36 60.51) (width 0.5) (layer "F.Cu") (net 7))
 (segment (start 46.34 60.53) (end 47.61 61.8) (width 0.5) (layer "F.Cu") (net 7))
 (segment (start 46.36 60.51) (end 46.34 60.53) (width 0.5) (layer "F.Cu") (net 7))
 (segment (start 47.61 61.8) (end 49.19 61.8) (width 0.5) (layer "F.Cu") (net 7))
 (segment (start 61.58 56.395) (end 61.58 57.355) (width 0.5) (layer "F.Cu") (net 16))
 (segment (start 61.58 57.355) (end 60.945 57.99) (width 0.5) (layer "F.Cu") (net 16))
 (segment (start 66.66 54.815) (end 63.16 54.815) (width 0.5) (layer "F.Cu") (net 16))
 (segment (start 63.16 54.815) (end 61.58 56.395) (width 0.5) (layer "F.Cu") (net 16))
 (segment (start 67.295 56.29) (end 67.295 55.45) (width 0.5) (layer "F.Cu") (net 16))
 (segment (start 67.295 55.45) (end 66.66 54.815) (width 0.5) (layer "F.Cu") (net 16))
 (segment (start 60.945 57.99) (end 59.545 57.99) (width 0.5) (layer "F.Cu") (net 16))
 (segment (start 61.58 59.26) (end 59.545 59.26) (width 0.5) (layer "F.Cu") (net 4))
 (segment (start 64.135 56.705) (end 61.58 59.26) (width 0.5) (layer "F.Cu") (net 4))
 (segment (start 64.135 56.29) (end 64.135 56.705) (width 0.5) (layer "F.Cu") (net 4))
 (segment (start 64.135 59.69) (end 64.135 62.11) (width 0.5) (layer "F.Cu") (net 3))
 (segment (start 67.295 59.69) (end 67.295 62.095) (width 0.5) (layer "F.Cu") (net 17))
 (segment (start 67.295 62.095) (end 67.31 62.11) (width 0.5) (layer "F.Cu") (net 17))
 (segment (start 62.215 63.07) (end 62.215 61.8) (width 0.5) (layer "F.Cu") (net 1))
 (segment (start 68.565 67.515) (end 69.835 66.245) (width 0.5) (layer "F.Cu") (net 1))
 (segment (start 48.88 73.23) (end 62.85 73.23) (width 0.5) (layer "F.Cu") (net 1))
 (segment (start 60.945 60.53) (end 59.545 60.53) (width 0.5) (layer "F.Cu") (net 1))
 (segment (start 69.835 64.34) (end 69.2 63.705) (width 0.5) (layer "F.Cu") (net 1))
 (segment (start 69.835 66.245) (end 69.835 64.34) (width 0.5) (layer "F.Cu") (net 1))
 (segment (start 64.755 67.515) (end 68.565 67.515) (width 0.5) (layer "F.Cu") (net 1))
 (segment (start 62.85 73.23) (end 62.85 69.42) (width 0.5) (layer "F.Cu") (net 1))
 (segment (start 62.85 69.42) (end 64.755 67.515) (width 0.5) (layer "F.Cu") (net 1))
 (segment (start 46.545 66.985) (end 49.19 64.34) (width 0.5) (layer "F.Cu") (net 1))
 (segment (start 62.85 63.705) (end 62.215 63.07) (width 0.5) (layer "F.Cu") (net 1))
 (segment (start 62.215 61.8) (end 60.945 60.53) (width 0.5) (layer "F.Cu") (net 1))
 (segment (start 46.545 69.42) (end 46.545 70.895) (width 0.5) (layer "F.Cu") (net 1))
 (segment (start 69.2 63.705) (end 62.85 63.705) (width 0.5) (layer "F.Cu") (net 1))
 (segment (start 46.545 69.42) (end 46.545 66.985) (width 0.5) (layer "F.Cu") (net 1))
 (segment (start 46.545 70.895) (end 48.88 73.23) (width 0.5) (layer "F.Cu") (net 1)))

